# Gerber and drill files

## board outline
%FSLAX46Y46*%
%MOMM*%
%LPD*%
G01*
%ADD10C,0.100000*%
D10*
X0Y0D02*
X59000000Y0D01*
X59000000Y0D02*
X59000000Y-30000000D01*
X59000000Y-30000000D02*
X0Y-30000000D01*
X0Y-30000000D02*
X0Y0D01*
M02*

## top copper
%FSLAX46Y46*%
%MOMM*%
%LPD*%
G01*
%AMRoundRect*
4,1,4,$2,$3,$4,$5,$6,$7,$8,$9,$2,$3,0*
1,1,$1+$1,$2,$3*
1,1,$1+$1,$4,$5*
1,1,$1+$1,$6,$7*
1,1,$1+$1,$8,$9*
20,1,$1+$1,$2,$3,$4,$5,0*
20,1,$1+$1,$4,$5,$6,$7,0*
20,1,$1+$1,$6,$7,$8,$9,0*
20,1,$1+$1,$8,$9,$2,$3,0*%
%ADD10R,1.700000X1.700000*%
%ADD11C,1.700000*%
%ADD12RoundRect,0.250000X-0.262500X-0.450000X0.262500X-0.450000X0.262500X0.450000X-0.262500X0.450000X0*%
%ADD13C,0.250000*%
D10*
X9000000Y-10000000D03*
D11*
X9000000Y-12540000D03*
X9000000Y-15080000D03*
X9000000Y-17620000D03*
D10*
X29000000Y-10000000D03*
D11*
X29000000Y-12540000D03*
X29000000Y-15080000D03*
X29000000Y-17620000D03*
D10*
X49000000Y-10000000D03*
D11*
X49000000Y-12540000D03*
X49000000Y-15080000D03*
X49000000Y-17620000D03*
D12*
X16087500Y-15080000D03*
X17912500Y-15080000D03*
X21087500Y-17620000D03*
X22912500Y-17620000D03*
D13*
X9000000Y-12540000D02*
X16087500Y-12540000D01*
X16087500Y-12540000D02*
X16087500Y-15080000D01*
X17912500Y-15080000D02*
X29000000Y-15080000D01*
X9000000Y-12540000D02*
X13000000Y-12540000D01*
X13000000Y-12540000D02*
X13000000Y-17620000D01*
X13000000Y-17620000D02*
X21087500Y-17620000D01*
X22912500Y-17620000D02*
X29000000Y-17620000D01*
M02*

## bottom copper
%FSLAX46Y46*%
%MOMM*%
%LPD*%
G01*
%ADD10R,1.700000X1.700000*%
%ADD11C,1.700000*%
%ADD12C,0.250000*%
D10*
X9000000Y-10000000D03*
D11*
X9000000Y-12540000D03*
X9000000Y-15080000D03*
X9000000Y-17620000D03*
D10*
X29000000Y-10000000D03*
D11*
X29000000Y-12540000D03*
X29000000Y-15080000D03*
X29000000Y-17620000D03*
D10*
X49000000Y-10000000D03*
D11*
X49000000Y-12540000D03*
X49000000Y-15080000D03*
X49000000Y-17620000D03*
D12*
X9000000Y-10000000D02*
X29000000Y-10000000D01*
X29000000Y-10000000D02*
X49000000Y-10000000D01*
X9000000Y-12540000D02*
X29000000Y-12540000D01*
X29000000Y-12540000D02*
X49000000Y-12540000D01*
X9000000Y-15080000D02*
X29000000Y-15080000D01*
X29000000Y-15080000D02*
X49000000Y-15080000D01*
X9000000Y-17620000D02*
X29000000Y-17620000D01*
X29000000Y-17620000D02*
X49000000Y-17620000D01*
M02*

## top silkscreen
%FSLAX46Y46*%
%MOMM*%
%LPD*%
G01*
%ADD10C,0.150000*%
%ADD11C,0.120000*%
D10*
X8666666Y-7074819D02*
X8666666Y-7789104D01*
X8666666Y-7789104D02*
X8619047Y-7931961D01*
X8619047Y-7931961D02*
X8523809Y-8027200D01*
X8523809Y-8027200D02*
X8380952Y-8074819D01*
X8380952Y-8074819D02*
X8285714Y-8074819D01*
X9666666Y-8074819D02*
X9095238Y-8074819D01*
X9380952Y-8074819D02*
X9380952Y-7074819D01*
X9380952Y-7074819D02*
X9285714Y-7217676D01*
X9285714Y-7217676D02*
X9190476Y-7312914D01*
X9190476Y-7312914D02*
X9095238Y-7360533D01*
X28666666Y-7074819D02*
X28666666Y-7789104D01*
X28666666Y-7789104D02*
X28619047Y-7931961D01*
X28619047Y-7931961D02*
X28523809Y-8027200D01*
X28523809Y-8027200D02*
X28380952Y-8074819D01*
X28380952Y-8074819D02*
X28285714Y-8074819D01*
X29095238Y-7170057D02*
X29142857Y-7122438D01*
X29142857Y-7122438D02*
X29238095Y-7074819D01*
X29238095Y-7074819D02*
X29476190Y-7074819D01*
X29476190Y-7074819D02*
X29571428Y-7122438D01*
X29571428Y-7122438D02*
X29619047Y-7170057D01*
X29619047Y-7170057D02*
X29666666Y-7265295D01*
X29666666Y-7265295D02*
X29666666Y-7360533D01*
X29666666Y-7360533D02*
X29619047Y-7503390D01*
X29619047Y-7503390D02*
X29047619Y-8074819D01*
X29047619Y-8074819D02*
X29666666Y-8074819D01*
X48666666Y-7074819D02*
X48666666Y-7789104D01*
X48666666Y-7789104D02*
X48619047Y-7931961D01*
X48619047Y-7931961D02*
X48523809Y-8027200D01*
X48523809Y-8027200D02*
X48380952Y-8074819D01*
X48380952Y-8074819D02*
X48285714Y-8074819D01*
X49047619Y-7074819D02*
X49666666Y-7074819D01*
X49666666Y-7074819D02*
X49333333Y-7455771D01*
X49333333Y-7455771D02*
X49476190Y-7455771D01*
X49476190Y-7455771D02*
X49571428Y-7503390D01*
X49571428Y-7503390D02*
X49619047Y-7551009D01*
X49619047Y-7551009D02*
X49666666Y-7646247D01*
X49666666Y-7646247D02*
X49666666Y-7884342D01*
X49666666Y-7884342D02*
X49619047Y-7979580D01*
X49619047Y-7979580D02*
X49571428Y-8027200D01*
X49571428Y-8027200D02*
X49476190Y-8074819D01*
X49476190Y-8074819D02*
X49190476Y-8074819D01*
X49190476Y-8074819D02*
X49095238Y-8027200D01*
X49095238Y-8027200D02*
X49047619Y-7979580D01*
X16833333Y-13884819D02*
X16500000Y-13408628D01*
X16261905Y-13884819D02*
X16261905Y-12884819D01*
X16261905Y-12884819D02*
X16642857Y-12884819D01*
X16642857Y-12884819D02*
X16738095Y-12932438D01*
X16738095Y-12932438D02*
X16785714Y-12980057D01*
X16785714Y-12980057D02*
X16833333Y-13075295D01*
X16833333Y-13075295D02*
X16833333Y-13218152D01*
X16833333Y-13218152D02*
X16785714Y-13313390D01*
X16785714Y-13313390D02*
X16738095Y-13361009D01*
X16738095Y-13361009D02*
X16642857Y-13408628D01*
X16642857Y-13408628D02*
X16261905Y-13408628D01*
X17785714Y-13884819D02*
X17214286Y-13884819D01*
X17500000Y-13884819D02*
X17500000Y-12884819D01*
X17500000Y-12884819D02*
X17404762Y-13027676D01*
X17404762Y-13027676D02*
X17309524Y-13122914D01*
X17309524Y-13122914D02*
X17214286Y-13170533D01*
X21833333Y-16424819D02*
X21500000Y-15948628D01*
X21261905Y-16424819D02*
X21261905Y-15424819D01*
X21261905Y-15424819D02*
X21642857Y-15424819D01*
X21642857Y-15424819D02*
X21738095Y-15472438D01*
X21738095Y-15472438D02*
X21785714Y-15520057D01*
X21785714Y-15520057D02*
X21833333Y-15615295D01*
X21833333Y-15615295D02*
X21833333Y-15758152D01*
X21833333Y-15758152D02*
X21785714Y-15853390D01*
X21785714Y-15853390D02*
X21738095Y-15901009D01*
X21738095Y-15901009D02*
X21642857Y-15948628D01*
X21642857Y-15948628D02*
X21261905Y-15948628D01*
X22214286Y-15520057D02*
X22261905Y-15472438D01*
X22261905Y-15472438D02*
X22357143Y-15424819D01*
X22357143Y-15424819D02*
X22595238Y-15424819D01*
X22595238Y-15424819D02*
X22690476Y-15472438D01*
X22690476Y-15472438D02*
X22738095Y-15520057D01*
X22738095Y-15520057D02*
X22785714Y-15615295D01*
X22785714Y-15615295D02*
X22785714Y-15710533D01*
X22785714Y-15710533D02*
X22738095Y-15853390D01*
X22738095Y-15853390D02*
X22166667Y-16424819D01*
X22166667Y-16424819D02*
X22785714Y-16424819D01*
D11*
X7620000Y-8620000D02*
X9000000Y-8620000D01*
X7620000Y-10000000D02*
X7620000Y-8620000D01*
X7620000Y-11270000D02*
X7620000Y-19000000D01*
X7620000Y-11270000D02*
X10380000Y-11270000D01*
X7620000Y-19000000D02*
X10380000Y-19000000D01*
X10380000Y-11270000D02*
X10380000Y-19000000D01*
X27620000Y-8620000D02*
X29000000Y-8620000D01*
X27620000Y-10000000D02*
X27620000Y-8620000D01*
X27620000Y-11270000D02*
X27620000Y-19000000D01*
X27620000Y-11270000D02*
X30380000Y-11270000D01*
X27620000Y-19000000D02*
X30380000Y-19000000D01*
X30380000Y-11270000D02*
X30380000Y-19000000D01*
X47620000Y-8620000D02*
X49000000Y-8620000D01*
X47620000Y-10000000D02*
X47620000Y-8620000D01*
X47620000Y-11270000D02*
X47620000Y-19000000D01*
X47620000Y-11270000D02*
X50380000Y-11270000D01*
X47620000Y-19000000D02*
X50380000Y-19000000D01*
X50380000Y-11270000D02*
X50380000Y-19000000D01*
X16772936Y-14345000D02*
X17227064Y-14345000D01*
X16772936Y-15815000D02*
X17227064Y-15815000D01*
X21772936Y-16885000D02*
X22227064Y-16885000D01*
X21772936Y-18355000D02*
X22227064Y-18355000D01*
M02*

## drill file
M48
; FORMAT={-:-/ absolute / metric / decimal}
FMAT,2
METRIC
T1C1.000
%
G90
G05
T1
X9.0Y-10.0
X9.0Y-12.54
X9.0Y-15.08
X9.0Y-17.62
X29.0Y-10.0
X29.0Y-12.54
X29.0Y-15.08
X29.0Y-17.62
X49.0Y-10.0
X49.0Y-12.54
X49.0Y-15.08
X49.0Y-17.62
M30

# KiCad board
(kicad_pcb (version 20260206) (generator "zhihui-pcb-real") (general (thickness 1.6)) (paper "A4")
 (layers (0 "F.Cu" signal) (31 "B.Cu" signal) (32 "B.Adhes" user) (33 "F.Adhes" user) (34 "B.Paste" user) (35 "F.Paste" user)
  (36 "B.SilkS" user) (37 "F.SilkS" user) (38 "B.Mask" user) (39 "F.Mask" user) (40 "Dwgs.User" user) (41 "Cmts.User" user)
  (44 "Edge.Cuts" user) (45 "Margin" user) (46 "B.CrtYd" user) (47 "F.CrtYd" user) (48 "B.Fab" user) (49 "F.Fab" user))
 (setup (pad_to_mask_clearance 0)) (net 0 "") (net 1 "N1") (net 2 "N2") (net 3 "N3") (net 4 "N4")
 (gr_line (start 0 0) (end 59 0) (stroke (width 0.1) (type default)) (layer "Edge.Cuts"))
 (gr_line (start 59 0) (end 59 30) (stroke (width 0.1) (type default)) (layer "Edge.Cuts"))
 (gr_line (start 59 30) (end 0 30) (stroke (width 0.1) (type default)) (layer "Edge.Cuts"))
 (gr_line (start 0 30) (end 0 0) (stroke (width 0.1) (type default)) (layer "Edge.Cuts"))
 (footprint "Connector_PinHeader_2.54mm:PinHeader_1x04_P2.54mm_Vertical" (layer "F.Cu")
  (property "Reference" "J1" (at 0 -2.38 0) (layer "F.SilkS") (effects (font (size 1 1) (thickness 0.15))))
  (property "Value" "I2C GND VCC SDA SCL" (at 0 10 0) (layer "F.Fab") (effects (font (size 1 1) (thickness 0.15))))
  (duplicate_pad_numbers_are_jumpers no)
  (fp_line (start -1.38 -1.38) (end 0 -1.38) (stroke (width 0.12) (type solid)) (layer "F.SilkS"))
  (fp_line (start -1.38 0) (end -1.38 -1.38) (stroke (width 0.12) (type solid)) (layer "F.SilkS"))
  (fp_line (start -1.38 1.27) (end -1.38 9) (stroke (width 0.12) (type solid)) (layer "F.SilkS"))
  (fp_line (start -1.38 1.27) (end 1.38 1.27) (stroke (width 0.12) (type solid)) (layer "F.SilkS"))
  (fp_line (start -1.38 9) (end 1.38 9) (stroke (width 0.12) (type solid)) (layer "F.SilkS"))
  (fp_line (start 1.38 1.27) (end 1.38 9) (stroke (width 0.12) (type solid)) (layer "F.SilkS"))
  (pad "1" thru_hole rect (at 0 0) (size 1.7 1.7) (drill 1) (layers "*.Cu" "*.Mask") (remove_unused_layers no) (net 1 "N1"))
  (pad "2" thru_hole circle (at 0 2.54) (size 1.7 1.7) (drill 1) (layers "*.Cu" "*.Mask") (remove_unused_layers no) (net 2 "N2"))
  (pad "3" thru_hole circle (at 0 5.08) (size 1.7 1.7) (drill 1) (layers "*.Cu" "*.Mask") (remove_unused_layers no) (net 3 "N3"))
  (pad "4" thru_hole circle (at 0 7.62) (size 1.7 1.7) (drill 1) (layers "*.Cu" "*.Mask") (remove_unused_layers no) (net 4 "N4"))
  (at 9 10 0))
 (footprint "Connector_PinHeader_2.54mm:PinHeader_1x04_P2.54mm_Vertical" (layer "F.Cu")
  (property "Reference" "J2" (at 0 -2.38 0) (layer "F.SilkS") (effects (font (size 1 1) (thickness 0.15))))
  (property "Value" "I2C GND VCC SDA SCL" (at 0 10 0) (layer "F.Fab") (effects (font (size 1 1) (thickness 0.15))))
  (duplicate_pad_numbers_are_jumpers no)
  (fp_line (start -1.38 -1.38) (end 0 -1.38) (stroke (width 0.12) (type solid)) (layer "F.SilkS"))
  (fp_line (start -1.38 0) (end -1.38 -1.38) (stroke (width 0.12) (type solid)) (layer "F.SilkS"))
  (fp_line (start -1.38 1.27) (end -1.38 9) (stroke (width 0.12) (type solid)) (layer "F.SilkS"))
  (fp_line (start -1.38 1.27) (end 1.38 1.27) (stroke (width 0.12) (type solid)) (layer "F.SilkS"))
  (fp_line (start -1.38 9) (end 1.38 9) (stroke (width 0.12) (type solid)) (layer "F.SilkS"))
  (fp_line (start 1.38 1.27) (end 1.38 9) (stroke (width 0.12) (type solid)) (layer "F.SilkS"))
  (pad "1" thru_hole rect (at 0 0) (size 1.7 1.7) (drill 1) (layers "*.Cu" "*.Mask") (remove_unused_layers no) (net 1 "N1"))
  (pad "2" thru_hole circle (at 0 2.54) (size 1.7 1.7) (drill 1) (layers "*.Cu" "*.Mask") (remove_unused_layers no) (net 2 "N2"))
  (pad "3" thru_hole circle (at 0 5.08) (size 1.7 1.7) (drill 1) (layers "*.Cu" "*.Mask") (remove_unused_layers no) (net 3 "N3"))
  (pad "4" thru_hole circle (at 0 7.62) (size 1.7 1.7) (drill 1) (layers "*.Cu" "*.Mask") (remove_unused_layers no) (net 4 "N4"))
  (at 29 10 0))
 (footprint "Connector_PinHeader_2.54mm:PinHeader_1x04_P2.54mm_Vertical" (layer "F.Cu")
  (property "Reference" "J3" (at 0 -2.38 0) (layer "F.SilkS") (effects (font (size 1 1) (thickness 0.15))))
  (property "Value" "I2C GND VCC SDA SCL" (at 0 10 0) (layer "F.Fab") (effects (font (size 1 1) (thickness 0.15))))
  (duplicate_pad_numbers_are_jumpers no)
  (fp_line (start -1.38 -1.38) (end 0 -1.38) (stroke (width 0.12) (type solid)) (layer "F.SilkS"))
  (fp_line (start -1.38 0) (end -1.38 -1.38) (stroke (width 0.12) (type solid)) (layer "F.SilkS"))
  (fp_line (start -1.38 1.27) (end -1.38 9) (stroke (width 0.12) (type solid)) (layer "F.SilkS"))
  (fp_line (start -1.38 1.27) (end 1.38 1.27) (stroke (width 0.12) (type solid)) (layer "F.SilkS"))
  (fp_line (start -1.38 9) (end 1.38 9) (stroke (width 0.12) (type solid)) (layer "F.SilkS"))
  (fp_line (start 1.38 1.27) (end 1.38 9) (stroke (width 0.12) (type solid)) (layer "F.SilkS"))
  (pad "1" thru_hole rect (at 0 0) (size 1.7 1.7) (drill 1) (layers "*.Cu" "*.Mask") (remove_unused_layers no) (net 1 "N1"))
  (pad "2" thru_hole circle (at 0 2.54) (size 1.7 1.7) (drill 1) (layers "*.Cu" "*.Mask") (remove_unused_layers no) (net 2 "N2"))
  (pad "3" thru_hole circle (at 0 5.08) (size 1.7 1.7) (drill 1) (layers "*.Cu" "*.Mask") (remove_unused_layers no) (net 3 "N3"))
  (pad "4" thru_hole circle (at 0 7.62) (size 1.7 1.7) (drill 1) (layers "*.Cu" "*.Mask") (remove_unused_layers no) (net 4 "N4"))
  (at 49 10 0))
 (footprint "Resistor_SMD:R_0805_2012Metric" (layer "F.Cu")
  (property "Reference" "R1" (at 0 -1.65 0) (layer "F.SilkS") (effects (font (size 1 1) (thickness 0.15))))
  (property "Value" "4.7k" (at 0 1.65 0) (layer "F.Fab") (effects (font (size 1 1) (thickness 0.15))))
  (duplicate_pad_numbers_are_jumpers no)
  (fp_line (start -0.227064 -0.735) (end 0.227064 -0.735) (stroke (width 0.12) (type solid)) (layer "F.SilkS"))
  (fp_line (start -0.227064 0.735) (end 0.227064 0.735) (stroke (width 0.12) (type solid)) (layer "F.SilkS"))
  (pad "1" smd roundrect (at -0.9125 0) (size 1.025 1.4) (layers "F.Cu" "F.Mask" "F.Paste") (roundrect_rratio 0.243902) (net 2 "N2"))
  (pad "2" smd roundrect (at 0.9125 0) (size 1.025 1.4) (layers "F.Cu" "F.Mask" "F.Paste") (roundrect_rratio 0.243902) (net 3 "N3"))
  (at 17 15.08 0))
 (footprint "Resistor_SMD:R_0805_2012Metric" (layer "F.Cu")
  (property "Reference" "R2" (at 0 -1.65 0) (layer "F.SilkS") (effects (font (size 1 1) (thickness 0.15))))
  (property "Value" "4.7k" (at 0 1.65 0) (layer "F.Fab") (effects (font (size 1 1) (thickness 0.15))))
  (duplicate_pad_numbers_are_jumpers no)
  (fp_line (start -0.227064 -0.735) (end 0.227064 -0.735) (stroke (width 0.12) (type solid)) (layer "F.SilkS"))
  (fp_line (start -0.227064 0.735) (end 0.227064 0.735) (stroke (width 0.12) (type solid)) (layer "F.SilkS"))
  (pad "1" smd roundrect (at -0.9125 0) (size 1.025 1.4) (layers "F.Cu" "F.Mask" "F.Paste") (roundrect_rratio 0.243902) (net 2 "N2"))
  (pad "2" smd roundrect (at 0.9125 0) (size 1.025 1.4) (layers "F.Cu" "F.Mask" "F.Paste") (roundrect_rratio 0.243902) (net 4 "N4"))
  (at 22 17.62 0))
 (segment (start 9 10) (end 29 10) (width 0.25) (layer "B.Cu") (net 1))
 (segment (start 29 10) (end 49 10) (width 0.25) (layer "B.Cu") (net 1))
 (segment (start 9 12.54) (end 29 12.54) (width 0.25) (layer "B.Cu") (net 2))
 (segment (start 29 12.54) (end 49 12.54) (width 0.25) (layer "B.Cu") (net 2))
 (segment (start 9 15.08) (end 29 15.08) (width 0.25) (layer "B.Cu") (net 3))
 (segment (start 29 15.08) (end 49 15.08) (width 0.25) (layer "B.Cu") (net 3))
 (segment (start 9 17.62) (end 29 17.62) (width 0.25) (layer "B.Cu") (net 4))
 (segment (start 29 17.62) (end 49 17.62) (width 0.25) (layer "B.Cu") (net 4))
 (segment (start 9 12.54) (end 16.0875 12.54) (width 0.25) (layer "F.Cu") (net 2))
 (segment (start 16.0875 12.54) (end 16.0875 15.08) (width 0.25) (layer "F.Cu") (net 2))
 (segment (start 17.9125 15.08) (end 29 15.08) (width 0.25) (layer "F.Cu") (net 3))
 (segment (start 9 12.54) (end 13 12.54) (width 0.25) (layer "F.Cu") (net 2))
 (segment (start 13 12.54) (end 13 17.62) (width 0.25) (layer "F.Cu") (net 2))
 (segment (start 13 17.62) (end 21.0875 17.62) (width 0.25) (layer "F.Cu") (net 2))
 (segment (start 22.9125 17.62) (end 29 17.62) (width 0.25) (layer "F.Cu") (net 4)))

